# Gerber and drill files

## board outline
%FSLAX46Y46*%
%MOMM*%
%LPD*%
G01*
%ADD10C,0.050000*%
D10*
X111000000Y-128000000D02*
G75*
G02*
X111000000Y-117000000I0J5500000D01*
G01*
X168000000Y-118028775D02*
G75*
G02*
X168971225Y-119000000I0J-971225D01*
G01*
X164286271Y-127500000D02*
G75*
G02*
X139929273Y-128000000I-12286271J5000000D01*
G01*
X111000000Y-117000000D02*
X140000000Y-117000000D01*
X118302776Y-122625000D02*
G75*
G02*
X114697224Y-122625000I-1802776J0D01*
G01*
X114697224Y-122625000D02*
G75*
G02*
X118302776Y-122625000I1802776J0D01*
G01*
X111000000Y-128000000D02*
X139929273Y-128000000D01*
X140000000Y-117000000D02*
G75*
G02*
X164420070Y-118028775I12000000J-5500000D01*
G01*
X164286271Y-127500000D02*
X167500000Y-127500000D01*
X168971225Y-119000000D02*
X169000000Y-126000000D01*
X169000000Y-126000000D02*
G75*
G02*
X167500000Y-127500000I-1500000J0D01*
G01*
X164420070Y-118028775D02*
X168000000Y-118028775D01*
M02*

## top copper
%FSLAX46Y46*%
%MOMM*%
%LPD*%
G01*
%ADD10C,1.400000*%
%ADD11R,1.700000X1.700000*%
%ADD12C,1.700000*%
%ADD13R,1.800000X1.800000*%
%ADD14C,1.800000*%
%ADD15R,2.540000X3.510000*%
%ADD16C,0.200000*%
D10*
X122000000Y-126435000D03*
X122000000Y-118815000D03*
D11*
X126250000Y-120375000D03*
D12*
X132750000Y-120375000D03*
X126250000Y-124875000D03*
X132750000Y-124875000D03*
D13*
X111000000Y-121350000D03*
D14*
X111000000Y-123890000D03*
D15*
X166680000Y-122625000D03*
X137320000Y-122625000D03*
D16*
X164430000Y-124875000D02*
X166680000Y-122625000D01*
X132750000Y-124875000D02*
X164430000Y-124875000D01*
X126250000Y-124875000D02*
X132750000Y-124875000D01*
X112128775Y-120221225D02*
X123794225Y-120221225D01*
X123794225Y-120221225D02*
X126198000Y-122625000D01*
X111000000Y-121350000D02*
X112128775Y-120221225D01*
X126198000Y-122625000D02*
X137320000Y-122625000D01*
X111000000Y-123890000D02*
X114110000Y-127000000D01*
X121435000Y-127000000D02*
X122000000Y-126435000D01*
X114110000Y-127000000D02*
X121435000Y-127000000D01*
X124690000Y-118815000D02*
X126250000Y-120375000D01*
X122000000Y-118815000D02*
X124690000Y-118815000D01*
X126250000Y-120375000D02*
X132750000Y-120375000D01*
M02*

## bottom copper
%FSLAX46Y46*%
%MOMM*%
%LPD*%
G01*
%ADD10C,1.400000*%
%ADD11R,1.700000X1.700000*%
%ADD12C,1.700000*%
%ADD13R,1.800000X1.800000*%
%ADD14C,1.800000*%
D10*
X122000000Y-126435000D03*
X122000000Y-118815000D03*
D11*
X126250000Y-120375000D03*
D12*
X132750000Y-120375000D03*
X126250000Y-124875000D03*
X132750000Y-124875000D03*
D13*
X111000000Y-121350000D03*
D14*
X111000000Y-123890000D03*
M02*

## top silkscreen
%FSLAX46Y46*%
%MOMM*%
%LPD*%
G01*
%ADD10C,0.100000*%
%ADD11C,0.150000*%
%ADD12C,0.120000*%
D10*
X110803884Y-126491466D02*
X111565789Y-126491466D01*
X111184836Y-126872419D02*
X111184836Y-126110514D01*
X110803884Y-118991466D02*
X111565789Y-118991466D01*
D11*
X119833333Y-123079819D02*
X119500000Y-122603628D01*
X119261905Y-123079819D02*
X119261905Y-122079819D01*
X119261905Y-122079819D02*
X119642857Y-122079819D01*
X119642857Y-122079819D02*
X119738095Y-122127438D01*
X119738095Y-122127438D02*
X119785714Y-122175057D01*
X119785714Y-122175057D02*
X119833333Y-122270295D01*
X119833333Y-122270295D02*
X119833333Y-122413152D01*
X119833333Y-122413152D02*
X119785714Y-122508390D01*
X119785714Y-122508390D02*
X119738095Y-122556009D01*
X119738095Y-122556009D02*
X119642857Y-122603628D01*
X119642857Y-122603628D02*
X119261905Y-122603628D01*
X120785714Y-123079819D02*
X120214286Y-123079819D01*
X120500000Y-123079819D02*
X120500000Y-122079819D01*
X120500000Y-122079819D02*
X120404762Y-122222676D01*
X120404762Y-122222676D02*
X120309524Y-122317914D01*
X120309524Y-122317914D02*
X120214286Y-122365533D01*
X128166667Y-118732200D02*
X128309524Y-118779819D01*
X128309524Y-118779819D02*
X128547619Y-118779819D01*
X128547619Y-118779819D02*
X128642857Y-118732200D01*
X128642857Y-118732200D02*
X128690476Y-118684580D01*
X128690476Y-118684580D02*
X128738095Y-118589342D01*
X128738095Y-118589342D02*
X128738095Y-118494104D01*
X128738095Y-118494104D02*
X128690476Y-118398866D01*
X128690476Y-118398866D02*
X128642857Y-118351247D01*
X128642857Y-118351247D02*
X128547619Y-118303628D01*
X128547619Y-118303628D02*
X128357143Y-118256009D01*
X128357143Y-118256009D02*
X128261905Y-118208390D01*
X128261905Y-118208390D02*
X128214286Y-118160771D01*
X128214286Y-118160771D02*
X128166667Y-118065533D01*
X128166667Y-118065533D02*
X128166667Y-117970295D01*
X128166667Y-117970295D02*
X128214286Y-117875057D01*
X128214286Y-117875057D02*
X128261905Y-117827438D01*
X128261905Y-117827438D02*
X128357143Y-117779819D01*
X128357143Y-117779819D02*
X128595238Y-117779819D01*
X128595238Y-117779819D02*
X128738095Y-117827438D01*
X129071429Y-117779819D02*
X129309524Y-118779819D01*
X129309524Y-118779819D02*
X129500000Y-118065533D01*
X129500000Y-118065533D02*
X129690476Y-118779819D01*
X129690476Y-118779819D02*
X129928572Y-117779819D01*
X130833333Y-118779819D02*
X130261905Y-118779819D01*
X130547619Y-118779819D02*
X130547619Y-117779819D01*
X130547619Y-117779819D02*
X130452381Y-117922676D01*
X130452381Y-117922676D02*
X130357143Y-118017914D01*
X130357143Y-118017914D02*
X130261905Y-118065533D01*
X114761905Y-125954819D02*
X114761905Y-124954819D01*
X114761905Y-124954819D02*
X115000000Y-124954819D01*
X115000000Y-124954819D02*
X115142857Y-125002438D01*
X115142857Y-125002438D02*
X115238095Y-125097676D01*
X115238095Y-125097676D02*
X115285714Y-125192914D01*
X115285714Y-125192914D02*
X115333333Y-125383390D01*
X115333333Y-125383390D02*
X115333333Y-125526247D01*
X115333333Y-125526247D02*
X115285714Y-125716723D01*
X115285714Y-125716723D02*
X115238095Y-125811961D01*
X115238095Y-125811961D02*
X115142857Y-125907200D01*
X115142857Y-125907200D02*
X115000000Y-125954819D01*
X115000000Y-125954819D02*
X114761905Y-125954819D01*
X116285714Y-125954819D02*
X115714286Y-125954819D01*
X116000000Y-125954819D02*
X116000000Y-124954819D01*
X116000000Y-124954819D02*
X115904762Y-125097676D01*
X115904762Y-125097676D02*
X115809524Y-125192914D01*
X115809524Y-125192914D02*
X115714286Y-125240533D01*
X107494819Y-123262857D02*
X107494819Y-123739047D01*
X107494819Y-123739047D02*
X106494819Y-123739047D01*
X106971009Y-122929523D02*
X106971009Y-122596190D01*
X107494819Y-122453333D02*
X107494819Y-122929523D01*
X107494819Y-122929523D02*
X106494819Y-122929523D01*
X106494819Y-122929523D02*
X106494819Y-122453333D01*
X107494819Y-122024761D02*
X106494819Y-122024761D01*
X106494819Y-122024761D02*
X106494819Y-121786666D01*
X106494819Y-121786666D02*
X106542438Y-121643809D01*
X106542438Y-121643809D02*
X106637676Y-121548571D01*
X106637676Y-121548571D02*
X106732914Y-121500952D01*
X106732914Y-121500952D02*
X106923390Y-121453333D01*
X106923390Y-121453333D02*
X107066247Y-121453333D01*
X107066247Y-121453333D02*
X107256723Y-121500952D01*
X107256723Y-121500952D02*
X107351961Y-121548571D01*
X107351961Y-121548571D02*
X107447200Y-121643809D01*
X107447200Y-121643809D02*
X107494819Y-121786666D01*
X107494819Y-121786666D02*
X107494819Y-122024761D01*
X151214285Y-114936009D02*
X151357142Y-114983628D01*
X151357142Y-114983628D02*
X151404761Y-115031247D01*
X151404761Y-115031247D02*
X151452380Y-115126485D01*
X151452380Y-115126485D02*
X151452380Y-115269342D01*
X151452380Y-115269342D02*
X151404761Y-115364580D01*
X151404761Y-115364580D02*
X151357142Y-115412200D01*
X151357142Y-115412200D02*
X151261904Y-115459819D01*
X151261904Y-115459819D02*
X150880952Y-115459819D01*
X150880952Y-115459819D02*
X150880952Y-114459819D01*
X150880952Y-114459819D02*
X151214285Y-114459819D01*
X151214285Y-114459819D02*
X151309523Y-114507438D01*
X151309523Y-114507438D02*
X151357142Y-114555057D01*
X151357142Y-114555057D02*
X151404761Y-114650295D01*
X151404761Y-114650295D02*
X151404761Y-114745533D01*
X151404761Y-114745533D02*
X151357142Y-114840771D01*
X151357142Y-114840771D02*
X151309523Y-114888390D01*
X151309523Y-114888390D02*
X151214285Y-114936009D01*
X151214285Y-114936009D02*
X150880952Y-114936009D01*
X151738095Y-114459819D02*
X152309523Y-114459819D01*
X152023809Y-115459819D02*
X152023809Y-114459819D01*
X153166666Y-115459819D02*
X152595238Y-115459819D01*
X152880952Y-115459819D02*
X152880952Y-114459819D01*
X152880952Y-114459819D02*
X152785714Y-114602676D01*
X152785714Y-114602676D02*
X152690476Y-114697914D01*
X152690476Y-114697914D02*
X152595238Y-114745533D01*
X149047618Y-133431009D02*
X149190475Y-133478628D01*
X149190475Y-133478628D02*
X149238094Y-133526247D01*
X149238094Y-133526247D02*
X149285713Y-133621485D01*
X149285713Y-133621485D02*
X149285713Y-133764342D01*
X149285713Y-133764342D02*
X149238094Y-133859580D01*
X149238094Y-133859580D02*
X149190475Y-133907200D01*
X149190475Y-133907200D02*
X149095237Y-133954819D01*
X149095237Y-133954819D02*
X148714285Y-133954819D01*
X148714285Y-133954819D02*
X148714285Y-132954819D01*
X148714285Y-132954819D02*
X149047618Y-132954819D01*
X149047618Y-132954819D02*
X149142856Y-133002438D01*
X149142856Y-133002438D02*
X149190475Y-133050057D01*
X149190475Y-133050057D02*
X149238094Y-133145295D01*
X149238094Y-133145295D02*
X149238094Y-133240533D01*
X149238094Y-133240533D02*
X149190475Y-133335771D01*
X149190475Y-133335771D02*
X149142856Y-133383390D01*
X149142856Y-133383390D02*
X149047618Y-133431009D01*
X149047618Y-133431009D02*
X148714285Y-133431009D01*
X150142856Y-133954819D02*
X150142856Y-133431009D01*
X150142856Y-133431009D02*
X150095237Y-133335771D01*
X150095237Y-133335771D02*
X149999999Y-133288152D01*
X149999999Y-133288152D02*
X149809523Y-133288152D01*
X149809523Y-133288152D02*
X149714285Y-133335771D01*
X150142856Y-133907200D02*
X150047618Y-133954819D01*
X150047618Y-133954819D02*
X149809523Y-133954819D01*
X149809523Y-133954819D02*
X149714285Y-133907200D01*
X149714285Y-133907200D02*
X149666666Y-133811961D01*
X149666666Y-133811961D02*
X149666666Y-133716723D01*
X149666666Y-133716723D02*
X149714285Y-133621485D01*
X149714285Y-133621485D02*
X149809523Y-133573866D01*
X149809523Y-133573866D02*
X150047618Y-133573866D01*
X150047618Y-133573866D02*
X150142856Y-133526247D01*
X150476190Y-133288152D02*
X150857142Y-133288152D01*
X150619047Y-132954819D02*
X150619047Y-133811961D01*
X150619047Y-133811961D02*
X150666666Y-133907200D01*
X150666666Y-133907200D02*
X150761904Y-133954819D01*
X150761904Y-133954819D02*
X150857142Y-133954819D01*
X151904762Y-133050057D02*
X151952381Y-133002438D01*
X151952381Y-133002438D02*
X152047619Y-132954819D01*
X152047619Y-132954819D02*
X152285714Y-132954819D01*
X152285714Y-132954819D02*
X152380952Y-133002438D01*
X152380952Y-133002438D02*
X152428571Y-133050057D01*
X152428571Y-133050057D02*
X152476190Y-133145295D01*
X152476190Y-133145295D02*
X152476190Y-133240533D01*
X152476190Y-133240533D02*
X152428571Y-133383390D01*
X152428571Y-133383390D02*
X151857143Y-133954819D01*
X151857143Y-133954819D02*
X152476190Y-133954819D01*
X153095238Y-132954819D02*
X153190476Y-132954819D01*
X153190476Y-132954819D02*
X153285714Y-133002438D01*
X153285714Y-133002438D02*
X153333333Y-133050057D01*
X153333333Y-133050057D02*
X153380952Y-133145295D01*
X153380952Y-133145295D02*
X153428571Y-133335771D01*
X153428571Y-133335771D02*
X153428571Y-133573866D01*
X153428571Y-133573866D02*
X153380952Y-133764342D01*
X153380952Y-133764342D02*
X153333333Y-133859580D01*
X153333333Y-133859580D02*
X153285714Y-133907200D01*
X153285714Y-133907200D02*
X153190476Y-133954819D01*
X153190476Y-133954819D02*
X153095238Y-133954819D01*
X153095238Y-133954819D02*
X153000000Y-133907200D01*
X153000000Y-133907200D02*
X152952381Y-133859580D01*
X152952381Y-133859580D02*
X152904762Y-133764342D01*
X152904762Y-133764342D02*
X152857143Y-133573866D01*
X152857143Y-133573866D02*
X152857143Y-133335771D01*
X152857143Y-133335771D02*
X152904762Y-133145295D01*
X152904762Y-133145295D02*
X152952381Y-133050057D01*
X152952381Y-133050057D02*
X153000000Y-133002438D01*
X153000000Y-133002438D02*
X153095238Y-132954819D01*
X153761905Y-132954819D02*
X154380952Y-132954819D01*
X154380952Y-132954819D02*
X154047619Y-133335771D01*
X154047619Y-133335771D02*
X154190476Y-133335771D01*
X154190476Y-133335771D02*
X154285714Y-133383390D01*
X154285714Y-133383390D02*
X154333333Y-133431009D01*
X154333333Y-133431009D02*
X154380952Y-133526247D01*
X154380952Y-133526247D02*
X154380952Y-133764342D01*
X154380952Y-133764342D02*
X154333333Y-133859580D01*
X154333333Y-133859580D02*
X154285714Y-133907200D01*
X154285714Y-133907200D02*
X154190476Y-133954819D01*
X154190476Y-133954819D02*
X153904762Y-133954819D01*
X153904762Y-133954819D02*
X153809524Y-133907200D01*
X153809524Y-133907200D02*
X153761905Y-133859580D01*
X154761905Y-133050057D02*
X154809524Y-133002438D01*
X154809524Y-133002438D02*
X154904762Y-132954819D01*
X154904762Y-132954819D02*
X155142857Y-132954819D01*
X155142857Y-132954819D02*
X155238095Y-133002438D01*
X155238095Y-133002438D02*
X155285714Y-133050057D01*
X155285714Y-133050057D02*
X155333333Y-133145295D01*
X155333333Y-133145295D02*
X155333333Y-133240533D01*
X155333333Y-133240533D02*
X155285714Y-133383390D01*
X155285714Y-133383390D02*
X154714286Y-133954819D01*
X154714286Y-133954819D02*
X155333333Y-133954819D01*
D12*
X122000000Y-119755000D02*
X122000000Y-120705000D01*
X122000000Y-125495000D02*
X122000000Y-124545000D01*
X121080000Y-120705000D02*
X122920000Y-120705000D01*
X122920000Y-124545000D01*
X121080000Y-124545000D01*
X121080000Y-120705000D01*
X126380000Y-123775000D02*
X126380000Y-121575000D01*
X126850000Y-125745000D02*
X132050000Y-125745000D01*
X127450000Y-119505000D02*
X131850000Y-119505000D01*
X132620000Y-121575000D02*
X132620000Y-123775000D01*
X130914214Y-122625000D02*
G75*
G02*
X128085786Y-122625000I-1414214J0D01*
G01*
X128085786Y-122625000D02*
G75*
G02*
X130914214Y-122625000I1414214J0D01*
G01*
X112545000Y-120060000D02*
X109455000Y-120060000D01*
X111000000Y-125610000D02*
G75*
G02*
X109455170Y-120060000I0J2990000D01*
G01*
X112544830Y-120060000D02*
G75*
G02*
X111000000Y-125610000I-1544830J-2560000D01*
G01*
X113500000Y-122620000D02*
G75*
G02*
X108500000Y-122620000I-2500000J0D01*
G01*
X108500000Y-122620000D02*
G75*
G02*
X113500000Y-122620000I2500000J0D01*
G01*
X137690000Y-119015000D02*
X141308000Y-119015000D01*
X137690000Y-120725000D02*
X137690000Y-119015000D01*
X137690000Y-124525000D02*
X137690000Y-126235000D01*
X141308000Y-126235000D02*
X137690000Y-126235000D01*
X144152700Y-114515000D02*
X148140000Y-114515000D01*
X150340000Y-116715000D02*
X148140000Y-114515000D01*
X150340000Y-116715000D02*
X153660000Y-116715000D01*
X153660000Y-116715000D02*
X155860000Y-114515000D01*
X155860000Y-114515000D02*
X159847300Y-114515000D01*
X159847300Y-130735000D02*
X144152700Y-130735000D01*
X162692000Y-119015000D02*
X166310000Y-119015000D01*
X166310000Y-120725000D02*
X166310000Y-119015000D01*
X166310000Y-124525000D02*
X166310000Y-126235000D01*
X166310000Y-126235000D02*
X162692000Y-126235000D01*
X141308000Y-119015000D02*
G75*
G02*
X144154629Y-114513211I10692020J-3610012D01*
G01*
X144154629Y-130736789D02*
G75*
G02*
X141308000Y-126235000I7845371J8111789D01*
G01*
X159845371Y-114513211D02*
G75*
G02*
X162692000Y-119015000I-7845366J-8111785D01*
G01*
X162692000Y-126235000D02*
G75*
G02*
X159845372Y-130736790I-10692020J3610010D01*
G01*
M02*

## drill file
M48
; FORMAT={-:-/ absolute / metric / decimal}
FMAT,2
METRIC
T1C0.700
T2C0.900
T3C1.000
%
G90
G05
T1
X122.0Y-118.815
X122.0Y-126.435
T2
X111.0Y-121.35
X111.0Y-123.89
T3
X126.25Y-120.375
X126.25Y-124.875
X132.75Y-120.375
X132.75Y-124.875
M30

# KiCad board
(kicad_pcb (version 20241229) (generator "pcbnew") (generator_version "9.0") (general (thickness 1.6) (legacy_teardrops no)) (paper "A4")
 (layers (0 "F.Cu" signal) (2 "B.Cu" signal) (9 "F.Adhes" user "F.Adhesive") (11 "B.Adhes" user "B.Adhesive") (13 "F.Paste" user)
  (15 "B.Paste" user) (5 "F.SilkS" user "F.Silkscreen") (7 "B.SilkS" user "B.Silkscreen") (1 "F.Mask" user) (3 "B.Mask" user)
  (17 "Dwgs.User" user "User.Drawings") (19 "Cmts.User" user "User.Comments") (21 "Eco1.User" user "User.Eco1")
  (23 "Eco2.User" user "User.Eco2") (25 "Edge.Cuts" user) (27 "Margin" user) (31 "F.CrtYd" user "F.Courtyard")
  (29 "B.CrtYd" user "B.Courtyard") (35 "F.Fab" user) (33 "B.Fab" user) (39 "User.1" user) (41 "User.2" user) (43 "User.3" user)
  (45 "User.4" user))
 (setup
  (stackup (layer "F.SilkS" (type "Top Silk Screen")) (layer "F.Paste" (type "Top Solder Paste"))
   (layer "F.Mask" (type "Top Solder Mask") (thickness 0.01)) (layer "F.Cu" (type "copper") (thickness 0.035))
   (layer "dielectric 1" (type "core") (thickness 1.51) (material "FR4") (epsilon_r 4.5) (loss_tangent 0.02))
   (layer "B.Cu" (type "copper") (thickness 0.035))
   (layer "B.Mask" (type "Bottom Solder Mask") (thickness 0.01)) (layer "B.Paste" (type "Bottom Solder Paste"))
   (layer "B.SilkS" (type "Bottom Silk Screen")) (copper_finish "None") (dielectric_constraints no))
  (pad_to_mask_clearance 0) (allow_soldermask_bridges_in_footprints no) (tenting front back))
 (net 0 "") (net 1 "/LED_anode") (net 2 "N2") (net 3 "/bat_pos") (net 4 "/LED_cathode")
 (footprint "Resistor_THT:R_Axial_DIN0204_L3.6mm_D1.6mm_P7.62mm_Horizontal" (layer "F.Cu") (at 122 126.435 90)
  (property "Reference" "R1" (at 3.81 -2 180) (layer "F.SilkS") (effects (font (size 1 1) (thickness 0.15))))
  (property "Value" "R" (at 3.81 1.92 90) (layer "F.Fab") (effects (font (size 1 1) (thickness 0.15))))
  (fp_line (start 6.68 0) (end 5.73 0) (stroke (width 0.12) (type solid)) (layer "F.SilkS"))
  (fp_line (start 0.94 0) (end 1.89 0) (stroke (width 0.12) (type solid)) (layer "F.SilkS"))
  (fp_rect (start 1.89 -0.92) (end 5.73 0.92) (stroke (width 0.12) (type solid)) (fill no) (layer "F.SilkS"))
  (pad "1" thru_hole circle (at 0 0 90) (size 1.4 1.4) (drill 0.7) (layers "*.Cu" "*.Mask") (remove_unused_layers no) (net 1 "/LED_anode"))
  (pad "2" thru_hole circle (at 7.62 0 90) (size 1.4 1.4) (drill 0.7) (layers "*.Cu" "*.Mask") (remove_unused_layers no) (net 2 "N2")))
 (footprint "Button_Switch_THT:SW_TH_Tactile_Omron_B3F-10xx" (layer "F.Cu") (at 126.25 120.375)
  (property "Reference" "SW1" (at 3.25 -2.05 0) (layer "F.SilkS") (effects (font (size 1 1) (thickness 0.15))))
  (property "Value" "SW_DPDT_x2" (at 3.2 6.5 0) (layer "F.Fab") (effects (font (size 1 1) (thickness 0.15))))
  (fp_line (start 0.13 3.4) (end 0.13 1.2) (stroke (width 0.12) (type solid)) (layer "F.SilkS"))
  (fp_line (start 0.6 5.37) (end 5.8 5.37) (stroke (width 0.12) (type solid)) (layer "F.SilkS"))
  (fp_line (start 1.2 -0.87) (end 5.6 -0.87) (stroke (width 0.12) (type solid)) (layer "F.SilkS"))
  (fp_line (start 6.37 1.2) (end 6.37 3.4) (stroke (width 0.12) (type solid)) (layer "F.SilkS"))
  (fp_circle (center 3.25 2.25) (end 4.25 3.25) (stroke (width 0.12) (type solid)) (fill no) (layer "F.SilkS"))
  (pad "1" thru_hole rect (at 0 0) (size 1.7 1.7) (drill 1) (layers "*.Cu" "*.Mask") (remove_unused_layers no) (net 2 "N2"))
  (pad "1" thru_hole circle (at 6.5 0) (size 1.7 1.7) (drill 1) (layers "*.Cu" "*.Mask") (remove_unused_layers no) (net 2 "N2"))
  (pad "2" thru_hole circle (at 0 4.5) (size 1.7 1.7) (drill 1) (layers "*.Cu" "*.Mask") (remove_unused_layers no) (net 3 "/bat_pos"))
  (pad "2" thru_hole circle (at 6.5 4.5) (size 1.7 1.7) (drill 1) (layers "*.Cu" "*.Mask") (remove_unused_layers no) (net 3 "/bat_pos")))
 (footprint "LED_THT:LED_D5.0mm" (layer "F.Cu") (at 111 121.35 -90)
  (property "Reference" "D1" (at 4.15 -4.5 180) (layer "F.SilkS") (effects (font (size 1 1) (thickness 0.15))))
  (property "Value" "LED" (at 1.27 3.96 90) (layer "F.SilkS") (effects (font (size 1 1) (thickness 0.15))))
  (fp_line (start -1.29 -1.545) (end -1.29 1.545) (stroke (width 0.12) (type solid)) (layer "F.SilkS"))
  (fp_arc (start 4.26 0) (mid 2.071779 2.880495) (end -1.29 1.54483) (stroke (width 0.12) (type solid)) (layer "F.SilkS"))
  (fp_arc (start -1.29 -1.54483) (mid 2.071779 -2.880495) (end 4.26 0) (stroke (width 0.12) (type solid)) (layer "F.SilkS"))
  (fp_circle (center 1.27 0) (end 3.77 0) (stroke (width 0.12) (type solid)) (fill no) (layer "F.SilkS"))
  (pad "1" thru_hole rect (at 0 0 270) (size 1.8 1.8) (drill 0.9) (layers "*.Cu" "*.Mask") (remove_unused_layers no) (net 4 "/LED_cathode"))
  (pad "2" thru_hole circle (at 2.54 0 270) (size 1.8 1.8) (drill 0.9) (layers "*.Cu" "*.Mask") (remove_unused_layers no)
   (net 1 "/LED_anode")))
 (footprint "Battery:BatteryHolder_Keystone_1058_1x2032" (layer "F.Cu") (at 152 122.625 180)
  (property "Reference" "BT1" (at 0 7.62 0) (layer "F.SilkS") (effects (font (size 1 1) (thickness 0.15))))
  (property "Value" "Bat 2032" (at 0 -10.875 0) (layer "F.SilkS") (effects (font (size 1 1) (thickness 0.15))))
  (fp_line (start 14.31 3.61) (end 10.692 3.61) (stroke (width 0.12) (type solid)) (layer "F.SilkS"))
  (fp_line (start 14.31 1.9) (end 14.31 3.61) (stroke (width 0.12) (type solid)) (layer "F.SilkS"))
  (fp_line (start 14.31 -1.9) (end 14.31 -3.61) (stroke (width 0.12) (type solid)) (layer "F.SilkS"))
  (fp_line (start 10.692 -3.61) (end 14.31 -3.61) (stroke (width 0.12) (type solid)) (layer "F.SilkS"))
  (fp_line (start 7.8473 8.11) (end 3.86 8.11) (stroke (width 0.12) (type solid)) (layer "F.SilkS"))
  (fp_line (start 1.66 5.91) (end 3.86 8.11) (stroke (width 0.12) (type solid)) (layer "F.SilkS"))
  (fp_line (start 1.66 5.91) (end -1.66 5.91) (stroke (width 0.12) (type solid)) (layer "F.SilkS"))
  (fp_line (start -1.66 5.91) (end -3.86 8.11) (stroke (width 0.12) (type solid)) (layer "F.SilkS"))
  (fp_line (start -3.86 8.11) (end -7.8473 8.11) (stroke (width 0.12) (type solid)) (layer "F.SilkS"))
  (fp_line (start -7.8473 -8.11) (end 7.8473 -8.11) (stroke (width 0.12) (type solid)) (layer "F.SilkS"))
  (fp_line (start -10.692 3.61) (end -14.31 3.61) (stroke (width 0.12) (type solid)) (layer "F.SilkS"))
  (fp_line (start -14.31 1.9) (end -14.31 3.61) (stroke (width 0.12) (type solid)) (layer "F.SilkS"))
  (fp_line (start -14.31 -1.9) (end -14.31 -3.61) (stroke (width 0.12) (type solid)) (layer "F.SilkS"))
  (fp_line (start -14.31 -3.61) (end -10.692 -3.61) (stroke (width 0.12) (type solid)) (layer "F.SilkS"))
  (fp_arc (start 10.692 3.61) (mid 9.538084 6.031244) (end 7.845371 8.111789) (stroke (width 0.12) (type solid)) (layer "F.SilkS"))
  (fp_arc (start 7.845371 -8.111789) (mid 9.538085 -6.031244) (end 10.692 -3.61) (stroke (width 0.12) (type solid)) (layer "F.SilkS"))
  (fp_arc (start -7.845371 8.111789) (mid -9.538085 6.031244) (end -10.692 3.61) (stroke (width 0.12) (type solid)) (layer "F.SilkS"))
  (fp_arc (start -10.692 -3.61) (mid -9.538084 -6.031244) (end -7.845371 -8.111789) (stroke (width 0.12) (type solid)) (layer "F.SilkS"))
  (pad "1" smd rect (at -14.68 0 180) (size 2.54 3.51) (layers "F.Cu" "F.Mask" "F.Paste") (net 3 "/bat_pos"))
  (pad "2" smd rect (at 14.68 0 180) (size 2.54 3.51) (layers "F.Cu" "F.Mask" "F.Paste") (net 4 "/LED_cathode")))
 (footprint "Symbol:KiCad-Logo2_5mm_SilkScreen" (layer "B.Cu") (at 152 121 180)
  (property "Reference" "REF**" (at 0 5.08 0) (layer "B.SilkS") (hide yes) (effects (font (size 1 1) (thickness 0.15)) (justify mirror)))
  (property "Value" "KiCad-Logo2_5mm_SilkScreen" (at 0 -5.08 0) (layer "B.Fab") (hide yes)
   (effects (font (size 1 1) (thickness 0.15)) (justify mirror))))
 (gr_arc (start 111 128) (mid 105.5 122.5) (end 111 117) (stroke (width 0.05) (type default)) (layer "Edge.Cuts"))
 (gr_arc (start 168 118.028775) (mid 168.68676 118.31324) (end 168.971225 119) (stroke (width 0.05) (type default)) (layer "Edge.Cuts"))
 (gr_arc (start 164.286271 127.5) (mid 152.27224 135.761913) (end 139.929273 128) (stroke (width 0.05) (type default)) (layer "Edge.Cuts"))
 (gr_line (start 111 117) (end 140 117) (stroke (width 0.05) (type default)) (layer "Edge.Cuts"))
 (gr_circle (center 116.5 122.625) (end 115 123.625) (stroke (width 0.05) (type default)) (fill no) (layer "Edge.Cuts"))
 (gr_line (start 111 128) (end 139.929273 128) (stroke (width 0.05) (type default)) (layer "Edge.Cuts"))
 (gr_arc (start 140 117) (mid 152.555616 109.31132) (end 164.42007 118.028775) (stroke (width 0.05) (type default)) (layer "Edge.Cuts"))
 (gr_line (start 164.286271 127.5) (end 167.5 127.5) (stroke (width 0.05) (type default)) (layer "Edge.Cuts"))
 (gr_line (start 168.971225 119) (end 169 126) (stroke (width 0.05) (type default)) (layer "Edge.Cuts"))
 (gr_arc (start 169 126) (mid 168.56066 127.06066) (end 167.5 127.5) (stroke (width 0.05) (type default)) (layer "Edge.Cuts"))
 (gr_line (start 164.42007 118.028775) (end 168 118.028775) (stroke (width 0.05) (type default)) (layer "Edge.Cuts"))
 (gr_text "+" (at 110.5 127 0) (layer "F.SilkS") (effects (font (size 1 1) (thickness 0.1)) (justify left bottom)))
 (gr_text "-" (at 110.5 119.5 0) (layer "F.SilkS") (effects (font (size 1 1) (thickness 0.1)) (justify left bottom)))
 (segment (start 164.43 124.875) (end 166.68 122.625) (width 0.2) (layer "F.Cu") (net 3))
 (segment (start 132.75 124.875) (end 164.43 124.875) (width 0.2) (layer "F.Cu") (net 3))
 (segment (start 126.25 124.875) (end 132.75 124.875) (width 0.2) (layer "F.Cu") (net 3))
 (segment (start 112.128775 120.221225) (end 123.794225 120.221225) (width 0.2) (layer "F.Cu") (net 4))
 (segment (start 123.794225 120.221225) (end 126.198 122.625) (width 0.2) (layer "F.Cu") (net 4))
 (segment (start 111 121.35) (end 112.128775 120.221225) (width 0.2) (layer "F.Cu") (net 4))
 (segment (start 126.198 122.625) (end 137.32 122.625) (width 0.2) (layer "F.Cu") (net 4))
 (segment (start 111 123.89) (end 114.11 127) (width 0.2) (layer "F.Cu") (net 1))
 (segment (start 121.435 127) (end 122 126.435) (width 0.2) (layer "F.Cu") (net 1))
 (segment (start 114.11 127) (end 121.435 127) (width 0.2) (layer "F.Cu") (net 1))
 (segment (start 124.69 118.815) (end 126.25 120.375) (width 0.2) (layer "F.Cu") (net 2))
 (segment (start 122 118.815) (end 124.69 118.815) (width 0.2) (layer "F.Cu") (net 2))
 (segment (start 126.25 120.375) (end 132.75 120.375) (width 0.2) (layer "F.Cu") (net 2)))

